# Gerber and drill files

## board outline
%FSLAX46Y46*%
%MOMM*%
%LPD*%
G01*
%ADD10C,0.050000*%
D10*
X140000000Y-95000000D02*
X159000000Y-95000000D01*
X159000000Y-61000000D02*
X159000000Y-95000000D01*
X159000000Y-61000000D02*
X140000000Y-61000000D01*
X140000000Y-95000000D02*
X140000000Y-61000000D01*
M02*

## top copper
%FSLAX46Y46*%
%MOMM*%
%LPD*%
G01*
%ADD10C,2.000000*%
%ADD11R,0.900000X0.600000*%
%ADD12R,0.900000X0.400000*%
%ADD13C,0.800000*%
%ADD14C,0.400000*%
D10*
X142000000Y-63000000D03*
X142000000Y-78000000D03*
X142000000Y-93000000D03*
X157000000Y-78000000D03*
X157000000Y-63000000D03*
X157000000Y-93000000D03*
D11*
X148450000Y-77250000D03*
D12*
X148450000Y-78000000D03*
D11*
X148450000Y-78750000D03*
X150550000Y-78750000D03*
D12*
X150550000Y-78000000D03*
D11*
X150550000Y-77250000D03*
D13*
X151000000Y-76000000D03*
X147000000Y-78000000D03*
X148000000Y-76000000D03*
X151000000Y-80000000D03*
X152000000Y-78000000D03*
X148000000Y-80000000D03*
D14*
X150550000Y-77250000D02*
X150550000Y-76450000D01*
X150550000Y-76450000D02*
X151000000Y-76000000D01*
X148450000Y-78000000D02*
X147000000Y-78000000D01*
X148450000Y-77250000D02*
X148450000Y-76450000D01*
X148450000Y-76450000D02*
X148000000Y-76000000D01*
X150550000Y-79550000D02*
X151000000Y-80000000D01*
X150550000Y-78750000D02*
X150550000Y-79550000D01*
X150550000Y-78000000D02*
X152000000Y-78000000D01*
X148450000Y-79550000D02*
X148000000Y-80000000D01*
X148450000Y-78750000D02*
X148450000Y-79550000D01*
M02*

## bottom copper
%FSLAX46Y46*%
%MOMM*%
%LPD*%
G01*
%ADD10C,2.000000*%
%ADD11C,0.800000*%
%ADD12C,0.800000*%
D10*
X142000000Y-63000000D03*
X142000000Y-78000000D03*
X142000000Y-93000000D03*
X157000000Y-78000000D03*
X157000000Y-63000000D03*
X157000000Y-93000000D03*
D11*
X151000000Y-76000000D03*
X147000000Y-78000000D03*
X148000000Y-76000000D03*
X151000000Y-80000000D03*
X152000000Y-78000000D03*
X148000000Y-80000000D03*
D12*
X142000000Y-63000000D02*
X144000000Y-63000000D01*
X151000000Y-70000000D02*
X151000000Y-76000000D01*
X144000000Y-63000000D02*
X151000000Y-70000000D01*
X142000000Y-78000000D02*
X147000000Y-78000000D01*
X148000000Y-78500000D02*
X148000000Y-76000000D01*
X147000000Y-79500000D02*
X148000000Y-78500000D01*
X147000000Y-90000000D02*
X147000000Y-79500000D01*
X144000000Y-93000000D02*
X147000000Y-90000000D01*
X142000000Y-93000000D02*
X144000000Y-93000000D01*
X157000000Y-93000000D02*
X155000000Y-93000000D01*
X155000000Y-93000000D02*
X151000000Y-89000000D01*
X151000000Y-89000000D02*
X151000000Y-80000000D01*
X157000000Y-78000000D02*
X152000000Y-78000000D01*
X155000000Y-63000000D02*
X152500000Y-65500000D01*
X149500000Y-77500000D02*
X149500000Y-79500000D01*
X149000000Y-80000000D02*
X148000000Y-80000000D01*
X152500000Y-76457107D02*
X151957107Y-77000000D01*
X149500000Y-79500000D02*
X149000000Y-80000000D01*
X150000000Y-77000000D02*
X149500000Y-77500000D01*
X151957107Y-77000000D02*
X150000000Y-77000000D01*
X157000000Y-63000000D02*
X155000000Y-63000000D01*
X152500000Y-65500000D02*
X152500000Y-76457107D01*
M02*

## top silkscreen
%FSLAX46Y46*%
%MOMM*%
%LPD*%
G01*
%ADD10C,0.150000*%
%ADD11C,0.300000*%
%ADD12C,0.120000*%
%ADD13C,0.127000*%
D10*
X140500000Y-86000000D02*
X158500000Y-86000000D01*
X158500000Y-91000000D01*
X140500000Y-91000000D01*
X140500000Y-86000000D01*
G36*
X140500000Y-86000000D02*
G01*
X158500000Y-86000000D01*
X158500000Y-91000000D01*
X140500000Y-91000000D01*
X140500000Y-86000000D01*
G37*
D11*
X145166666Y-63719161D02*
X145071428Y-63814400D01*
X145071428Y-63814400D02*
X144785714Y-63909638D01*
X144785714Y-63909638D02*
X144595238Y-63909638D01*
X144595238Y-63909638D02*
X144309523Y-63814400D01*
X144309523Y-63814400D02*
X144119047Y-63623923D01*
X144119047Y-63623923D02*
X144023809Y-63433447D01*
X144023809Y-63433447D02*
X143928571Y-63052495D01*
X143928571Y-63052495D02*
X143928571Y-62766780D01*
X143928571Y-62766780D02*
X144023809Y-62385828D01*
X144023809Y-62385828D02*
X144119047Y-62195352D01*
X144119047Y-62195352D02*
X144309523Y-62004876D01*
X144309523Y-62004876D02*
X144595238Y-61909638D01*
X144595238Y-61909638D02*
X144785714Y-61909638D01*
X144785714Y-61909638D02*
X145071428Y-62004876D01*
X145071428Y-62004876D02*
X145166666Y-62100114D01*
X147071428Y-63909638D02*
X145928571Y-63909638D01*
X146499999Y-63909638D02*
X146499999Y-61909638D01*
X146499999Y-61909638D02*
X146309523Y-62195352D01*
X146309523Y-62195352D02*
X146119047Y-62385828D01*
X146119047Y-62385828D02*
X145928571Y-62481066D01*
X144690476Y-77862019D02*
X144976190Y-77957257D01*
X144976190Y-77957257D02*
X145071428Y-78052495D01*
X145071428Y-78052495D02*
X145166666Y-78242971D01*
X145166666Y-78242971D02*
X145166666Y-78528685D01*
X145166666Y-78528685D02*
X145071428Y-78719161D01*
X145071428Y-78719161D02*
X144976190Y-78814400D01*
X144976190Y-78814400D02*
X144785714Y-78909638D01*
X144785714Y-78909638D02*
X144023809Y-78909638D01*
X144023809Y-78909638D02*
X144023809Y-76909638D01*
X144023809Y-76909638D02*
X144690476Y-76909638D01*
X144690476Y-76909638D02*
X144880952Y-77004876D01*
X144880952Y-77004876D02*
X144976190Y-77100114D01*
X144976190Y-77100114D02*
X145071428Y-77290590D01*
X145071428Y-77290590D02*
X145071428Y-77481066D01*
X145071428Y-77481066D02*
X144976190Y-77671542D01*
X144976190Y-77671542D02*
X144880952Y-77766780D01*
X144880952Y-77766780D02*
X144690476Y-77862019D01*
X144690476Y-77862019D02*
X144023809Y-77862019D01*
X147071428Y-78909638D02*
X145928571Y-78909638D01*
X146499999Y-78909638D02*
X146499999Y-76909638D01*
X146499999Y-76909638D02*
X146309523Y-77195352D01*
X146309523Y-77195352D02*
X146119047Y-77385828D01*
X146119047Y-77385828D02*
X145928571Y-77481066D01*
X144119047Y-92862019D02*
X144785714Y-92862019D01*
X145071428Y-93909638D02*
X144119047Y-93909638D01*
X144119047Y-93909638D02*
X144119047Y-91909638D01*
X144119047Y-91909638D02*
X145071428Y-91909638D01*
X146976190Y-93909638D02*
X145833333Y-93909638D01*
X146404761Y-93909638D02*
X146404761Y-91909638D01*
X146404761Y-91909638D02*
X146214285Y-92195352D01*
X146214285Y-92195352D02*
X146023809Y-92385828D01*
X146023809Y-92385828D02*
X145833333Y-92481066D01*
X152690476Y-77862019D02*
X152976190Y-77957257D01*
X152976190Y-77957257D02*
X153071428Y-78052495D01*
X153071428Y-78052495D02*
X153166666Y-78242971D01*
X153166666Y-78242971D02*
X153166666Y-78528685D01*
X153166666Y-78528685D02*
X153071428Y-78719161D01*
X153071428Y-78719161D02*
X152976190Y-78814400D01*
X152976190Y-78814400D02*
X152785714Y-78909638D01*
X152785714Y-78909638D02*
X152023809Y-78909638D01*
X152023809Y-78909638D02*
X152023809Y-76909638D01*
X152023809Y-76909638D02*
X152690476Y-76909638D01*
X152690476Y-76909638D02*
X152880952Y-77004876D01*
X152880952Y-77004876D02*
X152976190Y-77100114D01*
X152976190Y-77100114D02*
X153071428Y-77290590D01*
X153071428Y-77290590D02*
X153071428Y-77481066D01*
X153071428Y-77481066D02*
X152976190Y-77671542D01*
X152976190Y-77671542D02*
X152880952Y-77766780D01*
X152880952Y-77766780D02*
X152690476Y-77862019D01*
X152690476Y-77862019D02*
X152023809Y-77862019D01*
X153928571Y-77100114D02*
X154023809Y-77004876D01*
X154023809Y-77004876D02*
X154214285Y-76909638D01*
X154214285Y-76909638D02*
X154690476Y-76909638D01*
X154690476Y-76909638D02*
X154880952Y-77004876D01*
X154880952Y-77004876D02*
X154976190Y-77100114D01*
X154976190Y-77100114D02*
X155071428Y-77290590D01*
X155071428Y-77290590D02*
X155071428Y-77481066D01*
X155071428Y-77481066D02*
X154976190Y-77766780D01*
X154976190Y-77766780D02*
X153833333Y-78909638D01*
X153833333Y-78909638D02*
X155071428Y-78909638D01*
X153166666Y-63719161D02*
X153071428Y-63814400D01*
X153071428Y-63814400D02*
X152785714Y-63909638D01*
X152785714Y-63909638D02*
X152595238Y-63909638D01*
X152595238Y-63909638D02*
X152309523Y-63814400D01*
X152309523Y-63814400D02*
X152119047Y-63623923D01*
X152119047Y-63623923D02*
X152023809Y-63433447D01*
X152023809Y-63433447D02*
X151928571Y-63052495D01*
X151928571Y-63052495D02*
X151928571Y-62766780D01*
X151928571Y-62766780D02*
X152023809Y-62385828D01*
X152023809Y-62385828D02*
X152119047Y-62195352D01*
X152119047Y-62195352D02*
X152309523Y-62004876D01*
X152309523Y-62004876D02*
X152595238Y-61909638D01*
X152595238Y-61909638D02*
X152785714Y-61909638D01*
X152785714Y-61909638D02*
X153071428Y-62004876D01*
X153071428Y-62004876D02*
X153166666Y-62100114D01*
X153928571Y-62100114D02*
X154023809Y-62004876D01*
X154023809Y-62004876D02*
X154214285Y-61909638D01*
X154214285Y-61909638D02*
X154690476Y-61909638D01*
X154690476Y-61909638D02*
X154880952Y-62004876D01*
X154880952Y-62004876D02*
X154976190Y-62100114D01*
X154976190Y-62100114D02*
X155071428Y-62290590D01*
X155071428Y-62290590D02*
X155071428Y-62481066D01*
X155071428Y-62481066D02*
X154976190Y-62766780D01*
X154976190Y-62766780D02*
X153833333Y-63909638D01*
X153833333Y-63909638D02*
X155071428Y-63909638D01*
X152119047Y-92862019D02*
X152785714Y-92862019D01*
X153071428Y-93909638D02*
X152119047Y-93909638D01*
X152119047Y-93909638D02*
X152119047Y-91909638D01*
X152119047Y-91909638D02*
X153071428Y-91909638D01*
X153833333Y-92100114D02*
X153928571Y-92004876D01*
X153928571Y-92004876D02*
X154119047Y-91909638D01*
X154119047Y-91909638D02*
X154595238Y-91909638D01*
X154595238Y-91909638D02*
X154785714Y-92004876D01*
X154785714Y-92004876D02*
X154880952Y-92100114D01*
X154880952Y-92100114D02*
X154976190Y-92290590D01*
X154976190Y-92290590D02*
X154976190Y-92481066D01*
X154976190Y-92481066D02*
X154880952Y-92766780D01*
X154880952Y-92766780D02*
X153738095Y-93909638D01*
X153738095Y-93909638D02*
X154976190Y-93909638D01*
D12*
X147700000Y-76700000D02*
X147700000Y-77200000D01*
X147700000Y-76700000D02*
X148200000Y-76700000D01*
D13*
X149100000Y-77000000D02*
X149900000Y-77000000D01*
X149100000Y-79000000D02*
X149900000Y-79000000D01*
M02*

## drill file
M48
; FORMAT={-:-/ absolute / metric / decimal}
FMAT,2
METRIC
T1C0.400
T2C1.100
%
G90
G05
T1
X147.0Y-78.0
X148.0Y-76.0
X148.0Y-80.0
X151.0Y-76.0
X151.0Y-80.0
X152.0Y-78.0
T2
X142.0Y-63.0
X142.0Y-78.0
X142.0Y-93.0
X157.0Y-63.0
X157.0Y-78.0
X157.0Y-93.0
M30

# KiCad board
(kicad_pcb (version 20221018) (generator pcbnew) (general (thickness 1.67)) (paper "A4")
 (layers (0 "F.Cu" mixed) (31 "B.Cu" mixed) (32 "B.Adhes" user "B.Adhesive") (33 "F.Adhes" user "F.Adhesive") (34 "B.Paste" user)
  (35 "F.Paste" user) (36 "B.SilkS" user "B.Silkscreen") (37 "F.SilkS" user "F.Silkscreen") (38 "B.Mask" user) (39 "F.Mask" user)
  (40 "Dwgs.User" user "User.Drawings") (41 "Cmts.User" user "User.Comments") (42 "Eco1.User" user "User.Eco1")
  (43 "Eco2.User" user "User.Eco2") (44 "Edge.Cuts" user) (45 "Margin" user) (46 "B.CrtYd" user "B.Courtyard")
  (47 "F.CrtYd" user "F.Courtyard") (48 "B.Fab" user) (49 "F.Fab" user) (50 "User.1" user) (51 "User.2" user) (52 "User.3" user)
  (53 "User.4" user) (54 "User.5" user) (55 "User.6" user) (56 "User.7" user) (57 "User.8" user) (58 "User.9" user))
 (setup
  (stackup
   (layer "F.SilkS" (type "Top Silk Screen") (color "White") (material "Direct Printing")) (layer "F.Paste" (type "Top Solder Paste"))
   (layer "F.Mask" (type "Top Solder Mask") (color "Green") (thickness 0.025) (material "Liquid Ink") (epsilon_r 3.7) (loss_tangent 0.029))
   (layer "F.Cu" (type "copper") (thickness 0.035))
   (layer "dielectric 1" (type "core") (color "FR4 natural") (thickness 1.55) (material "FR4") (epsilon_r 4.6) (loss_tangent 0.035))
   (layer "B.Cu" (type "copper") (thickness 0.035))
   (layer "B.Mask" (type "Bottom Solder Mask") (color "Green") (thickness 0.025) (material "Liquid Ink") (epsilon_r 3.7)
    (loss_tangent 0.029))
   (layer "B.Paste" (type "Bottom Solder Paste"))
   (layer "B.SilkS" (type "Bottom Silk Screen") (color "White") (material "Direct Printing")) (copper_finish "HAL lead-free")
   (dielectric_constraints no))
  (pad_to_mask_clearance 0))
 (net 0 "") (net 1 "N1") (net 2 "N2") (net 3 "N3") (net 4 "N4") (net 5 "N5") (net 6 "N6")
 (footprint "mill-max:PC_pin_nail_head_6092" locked (layer "F.Cu") (at 142 63)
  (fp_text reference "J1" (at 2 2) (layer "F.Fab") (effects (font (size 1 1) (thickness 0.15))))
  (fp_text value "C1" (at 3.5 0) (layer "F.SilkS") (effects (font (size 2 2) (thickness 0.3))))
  (pad "1" thru_hole circle locked (at 0 0) (size 2 2) (drill 1.1) (layers "*.Cu" "*.Mask") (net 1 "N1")))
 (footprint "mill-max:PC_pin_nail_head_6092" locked (layer "F.Cu") (at 142 78)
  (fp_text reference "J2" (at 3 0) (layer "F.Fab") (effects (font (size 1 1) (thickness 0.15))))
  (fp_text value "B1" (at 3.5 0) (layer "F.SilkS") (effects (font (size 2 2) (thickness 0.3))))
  (pad "1" thru_hole circle locked (at 0 0) (size 2 2) (drill 1.1) (layers "*.Cu" "*.Mask") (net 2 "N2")))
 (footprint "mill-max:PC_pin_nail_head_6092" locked (layer "F.Cu") (at 142 93)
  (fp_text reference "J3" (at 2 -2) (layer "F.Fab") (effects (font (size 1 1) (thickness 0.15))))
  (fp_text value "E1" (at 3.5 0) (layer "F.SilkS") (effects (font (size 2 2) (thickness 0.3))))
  (pad "1" thru_hole circle locked (at 0 0) (size 2 2) (drill 1.1) (layers "*.Cu" "*.Mask") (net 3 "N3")))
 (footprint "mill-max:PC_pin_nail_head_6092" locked (layer "F.Cu") (at 157 78)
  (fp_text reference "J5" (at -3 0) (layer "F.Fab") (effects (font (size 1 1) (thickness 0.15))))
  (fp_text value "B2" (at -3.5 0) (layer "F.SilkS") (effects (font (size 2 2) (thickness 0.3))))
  (pad "1" thru_hole circle locked (at 0 0) (size 2 2) (drill 1.1) (layers "*.Cu" "*.Mask") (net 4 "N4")))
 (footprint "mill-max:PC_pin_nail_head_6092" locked (layer "F.Cu") (at 157 63)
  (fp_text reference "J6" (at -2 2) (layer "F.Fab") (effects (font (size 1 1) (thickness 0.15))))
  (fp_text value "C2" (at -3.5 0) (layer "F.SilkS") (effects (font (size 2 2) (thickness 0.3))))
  (pad "1" thru_hole circle locked (at 0 0) (size 2 2) (drill 1.1) (layers "*.Cu" "*.Mask") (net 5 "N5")))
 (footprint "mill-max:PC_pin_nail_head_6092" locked (layer "F.Cu") (at 157 93)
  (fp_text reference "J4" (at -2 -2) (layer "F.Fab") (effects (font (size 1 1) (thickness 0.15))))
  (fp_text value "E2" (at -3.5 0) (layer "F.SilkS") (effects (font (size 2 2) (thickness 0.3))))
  (pad "1" thru_hole circle locked (at 0 0) (size 2 2) (drill 1.1) (layers "*.Cu" "*.Mask") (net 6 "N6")))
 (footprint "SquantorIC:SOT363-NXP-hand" (layer "F.Cu") (at 149.5 78)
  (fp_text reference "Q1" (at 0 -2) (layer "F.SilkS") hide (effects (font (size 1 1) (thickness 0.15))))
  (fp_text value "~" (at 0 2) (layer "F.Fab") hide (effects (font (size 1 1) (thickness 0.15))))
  (fp_line (start -1.8 -1.3) (end -1.8 -0.8) (stroke (width 0.12) (type solid)) (layer "F.SilkS"))
  (fp_line (start -1.8 -1.3) (end -1.3 -1.3) (stroke (width 0.12) (type solid)) (layer "F.SilkS"))
  (fp_line (start -0.4 -1) (end 0.4 -1) (stroke (width 0.127) (type solid)) (layer "F.SilkS"))
  (fp_line (start -0.4 1) (end 0.4 1) (stroke (width 0.127) (type solid)) (layer "F.SilkS"))
  (pad "1" smd rect (at -1.05 -0.75 270) (size 0.6 0.9) (layers "F.Cu" "F.Paste" "F.Mask") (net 3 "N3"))
  (pad "2" smd rect (at -1.05 0 270) (size 0.4 0.9) (layers "F.Cu" "F.Paste" "F.Mask") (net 2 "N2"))
  (pad "3" smd rect (at -1.05 0.75 270) (size 0.6 0.9) (layers "F.Cu" "F.Paste" "F.Mask") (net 5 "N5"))
  (pad "4" smd rect (at 1.05 0.75 270) (size 0.6 0.9) (layers "F.Cu" "F.Paste" "F.Mask") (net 6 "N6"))
  (pad "5" smd rect (at 1.05 0 270) (size 0.4 0.9) (layers "F.Cu" "F.Paste" "F.Mask") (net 4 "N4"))
  (pad "6" smd rect (at 1.05 -0.75 270) (size 0.6 0.9) (layers "F.Cu" "F.Paste" "F.Mask") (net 1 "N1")))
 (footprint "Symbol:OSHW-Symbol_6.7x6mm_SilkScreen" (layer "B.Cu") (at 149 90 180)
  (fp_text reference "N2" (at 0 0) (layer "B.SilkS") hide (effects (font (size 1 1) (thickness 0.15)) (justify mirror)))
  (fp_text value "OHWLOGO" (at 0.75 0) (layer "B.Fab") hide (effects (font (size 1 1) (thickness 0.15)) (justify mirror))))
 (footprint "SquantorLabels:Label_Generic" (layer "B.Cu") (at 148.5 93.5)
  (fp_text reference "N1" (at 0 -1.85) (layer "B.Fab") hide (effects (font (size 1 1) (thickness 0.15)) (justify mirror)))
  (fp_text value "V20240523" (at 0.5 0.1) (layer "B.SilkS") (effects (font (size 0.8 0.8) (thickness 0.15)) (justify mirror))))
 (gr_rect (start 140.5 86) (end 158.5 91) (stroke (width 0.15) (type solid)) (fill solid) (layer "F.SilkS"))
 (gr_line (start 140 95) (end 159 95) (stroke (width 0.05) (type solid)) (layer "Edge.Cuts"))
 (gr_line (start 159 61) (end 159 95) (stroke (width 0.05) (type solid)) (layer "Edge.Cuts"))
 (gr_line (start 159 61) (end 140 61) (stroke (width 0.05) (type solid)) (layer "Edge.Cuts"))
 (gr_line (start 140 95) (end 140 61) (stroke (width 0.05) (type solid)) (layer "Edge.Cuts"))
 (segment (start 150.55 77.25) (end 150.55 76.45) (width 0.4) (layer "F.Cu") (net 1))
 (segment (start 150.55 76.45) (end 151 76) (width 0.4) (layer "F.Cu") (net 1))
 (via (at 151 76) (size 0.8) (drill 0.4) (layers "F.Cu" "B.Cu") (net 1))
 (segment (start 142 63) (end 144 63) (width 0.8) (layer "B.Cu") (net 1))
 (segment (start 151 70) (end 151 76) (width 0.8) (layer "B.Cu") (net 1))
 (segment (start 144 63) (end 151 70) (width 0.8) (layer "B.Cu") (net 1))
 (segment (start 148.45 78) (end 147 78) (width 0.4) (layer "F.Cu") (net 2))
 (via (at 147 78) (size 0.8) (drill 0.4) (layers "F.Cu" "B.Cu") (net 2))
 (segment (start 142 78) (end 147 78) (width 0.8) (layer "B.Cu") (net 2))
 (segment (start 148.45 77.25) (end 148.45 76.45) (width 0.4) (layer "F.Cu") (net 3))
 (segment (start 148.45 76.45) (end 148 76) (width 0.4) (layer "F.Cu") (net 3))
 (via (at 148 76) (size 0.8) (drill 0.4) (layers "F.Cu" "B.Cu") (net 3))
 (segment (start 148 78.5) (end 148 76) (width 0.8) (layer "B.Cu") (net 3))
 (segment (start 147 79.5) (end 148 78.5) (width 0.8) (layer "B.Cu") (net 3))
 (segment (start 147 90) (end 147 79.5) (width 0.8) (layer "B.Cu") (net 3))
 (segment (start 144 93) (end 147 90) (width 0.8) (layer "B.Cu") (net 3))
 (segment (start 142 93) (end 144 93) (width 0.8) (layer "B.Cu") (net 3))
 (segment (start 150.55 79.55) (end 151 80) (width 0.4) (layer "F.Cu") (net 6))
 (segment (start 150.55 78.75) (end 150.55 79.55) (width 0.4) (layer "F.Cu") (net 6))
 (via (at 151 80) (size 0.8) (drill 0.4) (layers "F.Cu" "B.Cu") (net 6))
 (segment (start 157 93) (end 155 93) (width 0.8) (layer "B.Cu") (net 6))
 (segment (start 155 93) (end 151 89) (width 0.8) (layer "B.Cu") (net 6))
 (segment (start 151 89) (end 151 80) (width 0.8) (layer "B.Cu") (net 6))
 (segment (start 150.55 78) (end 152 78) (width 0.4) (layer "F.Cu") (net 4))
 (via (at 152 78) (size 0.8) (drill 0.4) (layers "F.Cu" "B.Cu") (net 4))
 (segment (start 157 78) (end 152 78) (width 0.8) (layer "B.Cu") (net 4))
 (segment (start 148.45 79.55) (end 148 80) (width 0.4) (layer "F.Cu") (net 5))
 (segment (start 148.45 78.75) (end 148.45 79.55) (width 0.4) (layer "F.Cu") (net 5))
 (via (at 148 80) (size 0.8) (drill 0.4) (layers "F.Cu" "B.Cu") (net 5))
 (segment (start 155 63) (end 152.5 65.5) (width 0.8) (layer "B.Cu") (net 5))
 (segment (start 149.5 77.5) (end 149.5 79.5) (width 0.8) (layer "B.Cu") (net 5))
 (segment (start 149 80) (end 148 80) (width 0.8) (layer "B.Cu") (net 5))
 (segment (start 152.5 76.457107) (end 151.957107 77) (width 0.8) (layer "B.Cu") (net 5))
 (segment (start 149.5 79.5) (end 149 80) (width 0.8) (layer "B.Cu") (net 5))
 (segment (start 150 77) (end 149.5 77.5) (width 0.8) (layer "B.Cu") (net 5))
 (segment (start 151.957107 77) (end 150 77) (width 0.8) (layer "B.Cu") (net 5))
 (segment (start 157 63) (end 155 63) (width 0.8) (layer "B.Cu") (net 5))
 (segment (start 152.5 65.5) (end 152.5 76.457107) (width 0.8) (layer "B.Cu") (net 5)))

